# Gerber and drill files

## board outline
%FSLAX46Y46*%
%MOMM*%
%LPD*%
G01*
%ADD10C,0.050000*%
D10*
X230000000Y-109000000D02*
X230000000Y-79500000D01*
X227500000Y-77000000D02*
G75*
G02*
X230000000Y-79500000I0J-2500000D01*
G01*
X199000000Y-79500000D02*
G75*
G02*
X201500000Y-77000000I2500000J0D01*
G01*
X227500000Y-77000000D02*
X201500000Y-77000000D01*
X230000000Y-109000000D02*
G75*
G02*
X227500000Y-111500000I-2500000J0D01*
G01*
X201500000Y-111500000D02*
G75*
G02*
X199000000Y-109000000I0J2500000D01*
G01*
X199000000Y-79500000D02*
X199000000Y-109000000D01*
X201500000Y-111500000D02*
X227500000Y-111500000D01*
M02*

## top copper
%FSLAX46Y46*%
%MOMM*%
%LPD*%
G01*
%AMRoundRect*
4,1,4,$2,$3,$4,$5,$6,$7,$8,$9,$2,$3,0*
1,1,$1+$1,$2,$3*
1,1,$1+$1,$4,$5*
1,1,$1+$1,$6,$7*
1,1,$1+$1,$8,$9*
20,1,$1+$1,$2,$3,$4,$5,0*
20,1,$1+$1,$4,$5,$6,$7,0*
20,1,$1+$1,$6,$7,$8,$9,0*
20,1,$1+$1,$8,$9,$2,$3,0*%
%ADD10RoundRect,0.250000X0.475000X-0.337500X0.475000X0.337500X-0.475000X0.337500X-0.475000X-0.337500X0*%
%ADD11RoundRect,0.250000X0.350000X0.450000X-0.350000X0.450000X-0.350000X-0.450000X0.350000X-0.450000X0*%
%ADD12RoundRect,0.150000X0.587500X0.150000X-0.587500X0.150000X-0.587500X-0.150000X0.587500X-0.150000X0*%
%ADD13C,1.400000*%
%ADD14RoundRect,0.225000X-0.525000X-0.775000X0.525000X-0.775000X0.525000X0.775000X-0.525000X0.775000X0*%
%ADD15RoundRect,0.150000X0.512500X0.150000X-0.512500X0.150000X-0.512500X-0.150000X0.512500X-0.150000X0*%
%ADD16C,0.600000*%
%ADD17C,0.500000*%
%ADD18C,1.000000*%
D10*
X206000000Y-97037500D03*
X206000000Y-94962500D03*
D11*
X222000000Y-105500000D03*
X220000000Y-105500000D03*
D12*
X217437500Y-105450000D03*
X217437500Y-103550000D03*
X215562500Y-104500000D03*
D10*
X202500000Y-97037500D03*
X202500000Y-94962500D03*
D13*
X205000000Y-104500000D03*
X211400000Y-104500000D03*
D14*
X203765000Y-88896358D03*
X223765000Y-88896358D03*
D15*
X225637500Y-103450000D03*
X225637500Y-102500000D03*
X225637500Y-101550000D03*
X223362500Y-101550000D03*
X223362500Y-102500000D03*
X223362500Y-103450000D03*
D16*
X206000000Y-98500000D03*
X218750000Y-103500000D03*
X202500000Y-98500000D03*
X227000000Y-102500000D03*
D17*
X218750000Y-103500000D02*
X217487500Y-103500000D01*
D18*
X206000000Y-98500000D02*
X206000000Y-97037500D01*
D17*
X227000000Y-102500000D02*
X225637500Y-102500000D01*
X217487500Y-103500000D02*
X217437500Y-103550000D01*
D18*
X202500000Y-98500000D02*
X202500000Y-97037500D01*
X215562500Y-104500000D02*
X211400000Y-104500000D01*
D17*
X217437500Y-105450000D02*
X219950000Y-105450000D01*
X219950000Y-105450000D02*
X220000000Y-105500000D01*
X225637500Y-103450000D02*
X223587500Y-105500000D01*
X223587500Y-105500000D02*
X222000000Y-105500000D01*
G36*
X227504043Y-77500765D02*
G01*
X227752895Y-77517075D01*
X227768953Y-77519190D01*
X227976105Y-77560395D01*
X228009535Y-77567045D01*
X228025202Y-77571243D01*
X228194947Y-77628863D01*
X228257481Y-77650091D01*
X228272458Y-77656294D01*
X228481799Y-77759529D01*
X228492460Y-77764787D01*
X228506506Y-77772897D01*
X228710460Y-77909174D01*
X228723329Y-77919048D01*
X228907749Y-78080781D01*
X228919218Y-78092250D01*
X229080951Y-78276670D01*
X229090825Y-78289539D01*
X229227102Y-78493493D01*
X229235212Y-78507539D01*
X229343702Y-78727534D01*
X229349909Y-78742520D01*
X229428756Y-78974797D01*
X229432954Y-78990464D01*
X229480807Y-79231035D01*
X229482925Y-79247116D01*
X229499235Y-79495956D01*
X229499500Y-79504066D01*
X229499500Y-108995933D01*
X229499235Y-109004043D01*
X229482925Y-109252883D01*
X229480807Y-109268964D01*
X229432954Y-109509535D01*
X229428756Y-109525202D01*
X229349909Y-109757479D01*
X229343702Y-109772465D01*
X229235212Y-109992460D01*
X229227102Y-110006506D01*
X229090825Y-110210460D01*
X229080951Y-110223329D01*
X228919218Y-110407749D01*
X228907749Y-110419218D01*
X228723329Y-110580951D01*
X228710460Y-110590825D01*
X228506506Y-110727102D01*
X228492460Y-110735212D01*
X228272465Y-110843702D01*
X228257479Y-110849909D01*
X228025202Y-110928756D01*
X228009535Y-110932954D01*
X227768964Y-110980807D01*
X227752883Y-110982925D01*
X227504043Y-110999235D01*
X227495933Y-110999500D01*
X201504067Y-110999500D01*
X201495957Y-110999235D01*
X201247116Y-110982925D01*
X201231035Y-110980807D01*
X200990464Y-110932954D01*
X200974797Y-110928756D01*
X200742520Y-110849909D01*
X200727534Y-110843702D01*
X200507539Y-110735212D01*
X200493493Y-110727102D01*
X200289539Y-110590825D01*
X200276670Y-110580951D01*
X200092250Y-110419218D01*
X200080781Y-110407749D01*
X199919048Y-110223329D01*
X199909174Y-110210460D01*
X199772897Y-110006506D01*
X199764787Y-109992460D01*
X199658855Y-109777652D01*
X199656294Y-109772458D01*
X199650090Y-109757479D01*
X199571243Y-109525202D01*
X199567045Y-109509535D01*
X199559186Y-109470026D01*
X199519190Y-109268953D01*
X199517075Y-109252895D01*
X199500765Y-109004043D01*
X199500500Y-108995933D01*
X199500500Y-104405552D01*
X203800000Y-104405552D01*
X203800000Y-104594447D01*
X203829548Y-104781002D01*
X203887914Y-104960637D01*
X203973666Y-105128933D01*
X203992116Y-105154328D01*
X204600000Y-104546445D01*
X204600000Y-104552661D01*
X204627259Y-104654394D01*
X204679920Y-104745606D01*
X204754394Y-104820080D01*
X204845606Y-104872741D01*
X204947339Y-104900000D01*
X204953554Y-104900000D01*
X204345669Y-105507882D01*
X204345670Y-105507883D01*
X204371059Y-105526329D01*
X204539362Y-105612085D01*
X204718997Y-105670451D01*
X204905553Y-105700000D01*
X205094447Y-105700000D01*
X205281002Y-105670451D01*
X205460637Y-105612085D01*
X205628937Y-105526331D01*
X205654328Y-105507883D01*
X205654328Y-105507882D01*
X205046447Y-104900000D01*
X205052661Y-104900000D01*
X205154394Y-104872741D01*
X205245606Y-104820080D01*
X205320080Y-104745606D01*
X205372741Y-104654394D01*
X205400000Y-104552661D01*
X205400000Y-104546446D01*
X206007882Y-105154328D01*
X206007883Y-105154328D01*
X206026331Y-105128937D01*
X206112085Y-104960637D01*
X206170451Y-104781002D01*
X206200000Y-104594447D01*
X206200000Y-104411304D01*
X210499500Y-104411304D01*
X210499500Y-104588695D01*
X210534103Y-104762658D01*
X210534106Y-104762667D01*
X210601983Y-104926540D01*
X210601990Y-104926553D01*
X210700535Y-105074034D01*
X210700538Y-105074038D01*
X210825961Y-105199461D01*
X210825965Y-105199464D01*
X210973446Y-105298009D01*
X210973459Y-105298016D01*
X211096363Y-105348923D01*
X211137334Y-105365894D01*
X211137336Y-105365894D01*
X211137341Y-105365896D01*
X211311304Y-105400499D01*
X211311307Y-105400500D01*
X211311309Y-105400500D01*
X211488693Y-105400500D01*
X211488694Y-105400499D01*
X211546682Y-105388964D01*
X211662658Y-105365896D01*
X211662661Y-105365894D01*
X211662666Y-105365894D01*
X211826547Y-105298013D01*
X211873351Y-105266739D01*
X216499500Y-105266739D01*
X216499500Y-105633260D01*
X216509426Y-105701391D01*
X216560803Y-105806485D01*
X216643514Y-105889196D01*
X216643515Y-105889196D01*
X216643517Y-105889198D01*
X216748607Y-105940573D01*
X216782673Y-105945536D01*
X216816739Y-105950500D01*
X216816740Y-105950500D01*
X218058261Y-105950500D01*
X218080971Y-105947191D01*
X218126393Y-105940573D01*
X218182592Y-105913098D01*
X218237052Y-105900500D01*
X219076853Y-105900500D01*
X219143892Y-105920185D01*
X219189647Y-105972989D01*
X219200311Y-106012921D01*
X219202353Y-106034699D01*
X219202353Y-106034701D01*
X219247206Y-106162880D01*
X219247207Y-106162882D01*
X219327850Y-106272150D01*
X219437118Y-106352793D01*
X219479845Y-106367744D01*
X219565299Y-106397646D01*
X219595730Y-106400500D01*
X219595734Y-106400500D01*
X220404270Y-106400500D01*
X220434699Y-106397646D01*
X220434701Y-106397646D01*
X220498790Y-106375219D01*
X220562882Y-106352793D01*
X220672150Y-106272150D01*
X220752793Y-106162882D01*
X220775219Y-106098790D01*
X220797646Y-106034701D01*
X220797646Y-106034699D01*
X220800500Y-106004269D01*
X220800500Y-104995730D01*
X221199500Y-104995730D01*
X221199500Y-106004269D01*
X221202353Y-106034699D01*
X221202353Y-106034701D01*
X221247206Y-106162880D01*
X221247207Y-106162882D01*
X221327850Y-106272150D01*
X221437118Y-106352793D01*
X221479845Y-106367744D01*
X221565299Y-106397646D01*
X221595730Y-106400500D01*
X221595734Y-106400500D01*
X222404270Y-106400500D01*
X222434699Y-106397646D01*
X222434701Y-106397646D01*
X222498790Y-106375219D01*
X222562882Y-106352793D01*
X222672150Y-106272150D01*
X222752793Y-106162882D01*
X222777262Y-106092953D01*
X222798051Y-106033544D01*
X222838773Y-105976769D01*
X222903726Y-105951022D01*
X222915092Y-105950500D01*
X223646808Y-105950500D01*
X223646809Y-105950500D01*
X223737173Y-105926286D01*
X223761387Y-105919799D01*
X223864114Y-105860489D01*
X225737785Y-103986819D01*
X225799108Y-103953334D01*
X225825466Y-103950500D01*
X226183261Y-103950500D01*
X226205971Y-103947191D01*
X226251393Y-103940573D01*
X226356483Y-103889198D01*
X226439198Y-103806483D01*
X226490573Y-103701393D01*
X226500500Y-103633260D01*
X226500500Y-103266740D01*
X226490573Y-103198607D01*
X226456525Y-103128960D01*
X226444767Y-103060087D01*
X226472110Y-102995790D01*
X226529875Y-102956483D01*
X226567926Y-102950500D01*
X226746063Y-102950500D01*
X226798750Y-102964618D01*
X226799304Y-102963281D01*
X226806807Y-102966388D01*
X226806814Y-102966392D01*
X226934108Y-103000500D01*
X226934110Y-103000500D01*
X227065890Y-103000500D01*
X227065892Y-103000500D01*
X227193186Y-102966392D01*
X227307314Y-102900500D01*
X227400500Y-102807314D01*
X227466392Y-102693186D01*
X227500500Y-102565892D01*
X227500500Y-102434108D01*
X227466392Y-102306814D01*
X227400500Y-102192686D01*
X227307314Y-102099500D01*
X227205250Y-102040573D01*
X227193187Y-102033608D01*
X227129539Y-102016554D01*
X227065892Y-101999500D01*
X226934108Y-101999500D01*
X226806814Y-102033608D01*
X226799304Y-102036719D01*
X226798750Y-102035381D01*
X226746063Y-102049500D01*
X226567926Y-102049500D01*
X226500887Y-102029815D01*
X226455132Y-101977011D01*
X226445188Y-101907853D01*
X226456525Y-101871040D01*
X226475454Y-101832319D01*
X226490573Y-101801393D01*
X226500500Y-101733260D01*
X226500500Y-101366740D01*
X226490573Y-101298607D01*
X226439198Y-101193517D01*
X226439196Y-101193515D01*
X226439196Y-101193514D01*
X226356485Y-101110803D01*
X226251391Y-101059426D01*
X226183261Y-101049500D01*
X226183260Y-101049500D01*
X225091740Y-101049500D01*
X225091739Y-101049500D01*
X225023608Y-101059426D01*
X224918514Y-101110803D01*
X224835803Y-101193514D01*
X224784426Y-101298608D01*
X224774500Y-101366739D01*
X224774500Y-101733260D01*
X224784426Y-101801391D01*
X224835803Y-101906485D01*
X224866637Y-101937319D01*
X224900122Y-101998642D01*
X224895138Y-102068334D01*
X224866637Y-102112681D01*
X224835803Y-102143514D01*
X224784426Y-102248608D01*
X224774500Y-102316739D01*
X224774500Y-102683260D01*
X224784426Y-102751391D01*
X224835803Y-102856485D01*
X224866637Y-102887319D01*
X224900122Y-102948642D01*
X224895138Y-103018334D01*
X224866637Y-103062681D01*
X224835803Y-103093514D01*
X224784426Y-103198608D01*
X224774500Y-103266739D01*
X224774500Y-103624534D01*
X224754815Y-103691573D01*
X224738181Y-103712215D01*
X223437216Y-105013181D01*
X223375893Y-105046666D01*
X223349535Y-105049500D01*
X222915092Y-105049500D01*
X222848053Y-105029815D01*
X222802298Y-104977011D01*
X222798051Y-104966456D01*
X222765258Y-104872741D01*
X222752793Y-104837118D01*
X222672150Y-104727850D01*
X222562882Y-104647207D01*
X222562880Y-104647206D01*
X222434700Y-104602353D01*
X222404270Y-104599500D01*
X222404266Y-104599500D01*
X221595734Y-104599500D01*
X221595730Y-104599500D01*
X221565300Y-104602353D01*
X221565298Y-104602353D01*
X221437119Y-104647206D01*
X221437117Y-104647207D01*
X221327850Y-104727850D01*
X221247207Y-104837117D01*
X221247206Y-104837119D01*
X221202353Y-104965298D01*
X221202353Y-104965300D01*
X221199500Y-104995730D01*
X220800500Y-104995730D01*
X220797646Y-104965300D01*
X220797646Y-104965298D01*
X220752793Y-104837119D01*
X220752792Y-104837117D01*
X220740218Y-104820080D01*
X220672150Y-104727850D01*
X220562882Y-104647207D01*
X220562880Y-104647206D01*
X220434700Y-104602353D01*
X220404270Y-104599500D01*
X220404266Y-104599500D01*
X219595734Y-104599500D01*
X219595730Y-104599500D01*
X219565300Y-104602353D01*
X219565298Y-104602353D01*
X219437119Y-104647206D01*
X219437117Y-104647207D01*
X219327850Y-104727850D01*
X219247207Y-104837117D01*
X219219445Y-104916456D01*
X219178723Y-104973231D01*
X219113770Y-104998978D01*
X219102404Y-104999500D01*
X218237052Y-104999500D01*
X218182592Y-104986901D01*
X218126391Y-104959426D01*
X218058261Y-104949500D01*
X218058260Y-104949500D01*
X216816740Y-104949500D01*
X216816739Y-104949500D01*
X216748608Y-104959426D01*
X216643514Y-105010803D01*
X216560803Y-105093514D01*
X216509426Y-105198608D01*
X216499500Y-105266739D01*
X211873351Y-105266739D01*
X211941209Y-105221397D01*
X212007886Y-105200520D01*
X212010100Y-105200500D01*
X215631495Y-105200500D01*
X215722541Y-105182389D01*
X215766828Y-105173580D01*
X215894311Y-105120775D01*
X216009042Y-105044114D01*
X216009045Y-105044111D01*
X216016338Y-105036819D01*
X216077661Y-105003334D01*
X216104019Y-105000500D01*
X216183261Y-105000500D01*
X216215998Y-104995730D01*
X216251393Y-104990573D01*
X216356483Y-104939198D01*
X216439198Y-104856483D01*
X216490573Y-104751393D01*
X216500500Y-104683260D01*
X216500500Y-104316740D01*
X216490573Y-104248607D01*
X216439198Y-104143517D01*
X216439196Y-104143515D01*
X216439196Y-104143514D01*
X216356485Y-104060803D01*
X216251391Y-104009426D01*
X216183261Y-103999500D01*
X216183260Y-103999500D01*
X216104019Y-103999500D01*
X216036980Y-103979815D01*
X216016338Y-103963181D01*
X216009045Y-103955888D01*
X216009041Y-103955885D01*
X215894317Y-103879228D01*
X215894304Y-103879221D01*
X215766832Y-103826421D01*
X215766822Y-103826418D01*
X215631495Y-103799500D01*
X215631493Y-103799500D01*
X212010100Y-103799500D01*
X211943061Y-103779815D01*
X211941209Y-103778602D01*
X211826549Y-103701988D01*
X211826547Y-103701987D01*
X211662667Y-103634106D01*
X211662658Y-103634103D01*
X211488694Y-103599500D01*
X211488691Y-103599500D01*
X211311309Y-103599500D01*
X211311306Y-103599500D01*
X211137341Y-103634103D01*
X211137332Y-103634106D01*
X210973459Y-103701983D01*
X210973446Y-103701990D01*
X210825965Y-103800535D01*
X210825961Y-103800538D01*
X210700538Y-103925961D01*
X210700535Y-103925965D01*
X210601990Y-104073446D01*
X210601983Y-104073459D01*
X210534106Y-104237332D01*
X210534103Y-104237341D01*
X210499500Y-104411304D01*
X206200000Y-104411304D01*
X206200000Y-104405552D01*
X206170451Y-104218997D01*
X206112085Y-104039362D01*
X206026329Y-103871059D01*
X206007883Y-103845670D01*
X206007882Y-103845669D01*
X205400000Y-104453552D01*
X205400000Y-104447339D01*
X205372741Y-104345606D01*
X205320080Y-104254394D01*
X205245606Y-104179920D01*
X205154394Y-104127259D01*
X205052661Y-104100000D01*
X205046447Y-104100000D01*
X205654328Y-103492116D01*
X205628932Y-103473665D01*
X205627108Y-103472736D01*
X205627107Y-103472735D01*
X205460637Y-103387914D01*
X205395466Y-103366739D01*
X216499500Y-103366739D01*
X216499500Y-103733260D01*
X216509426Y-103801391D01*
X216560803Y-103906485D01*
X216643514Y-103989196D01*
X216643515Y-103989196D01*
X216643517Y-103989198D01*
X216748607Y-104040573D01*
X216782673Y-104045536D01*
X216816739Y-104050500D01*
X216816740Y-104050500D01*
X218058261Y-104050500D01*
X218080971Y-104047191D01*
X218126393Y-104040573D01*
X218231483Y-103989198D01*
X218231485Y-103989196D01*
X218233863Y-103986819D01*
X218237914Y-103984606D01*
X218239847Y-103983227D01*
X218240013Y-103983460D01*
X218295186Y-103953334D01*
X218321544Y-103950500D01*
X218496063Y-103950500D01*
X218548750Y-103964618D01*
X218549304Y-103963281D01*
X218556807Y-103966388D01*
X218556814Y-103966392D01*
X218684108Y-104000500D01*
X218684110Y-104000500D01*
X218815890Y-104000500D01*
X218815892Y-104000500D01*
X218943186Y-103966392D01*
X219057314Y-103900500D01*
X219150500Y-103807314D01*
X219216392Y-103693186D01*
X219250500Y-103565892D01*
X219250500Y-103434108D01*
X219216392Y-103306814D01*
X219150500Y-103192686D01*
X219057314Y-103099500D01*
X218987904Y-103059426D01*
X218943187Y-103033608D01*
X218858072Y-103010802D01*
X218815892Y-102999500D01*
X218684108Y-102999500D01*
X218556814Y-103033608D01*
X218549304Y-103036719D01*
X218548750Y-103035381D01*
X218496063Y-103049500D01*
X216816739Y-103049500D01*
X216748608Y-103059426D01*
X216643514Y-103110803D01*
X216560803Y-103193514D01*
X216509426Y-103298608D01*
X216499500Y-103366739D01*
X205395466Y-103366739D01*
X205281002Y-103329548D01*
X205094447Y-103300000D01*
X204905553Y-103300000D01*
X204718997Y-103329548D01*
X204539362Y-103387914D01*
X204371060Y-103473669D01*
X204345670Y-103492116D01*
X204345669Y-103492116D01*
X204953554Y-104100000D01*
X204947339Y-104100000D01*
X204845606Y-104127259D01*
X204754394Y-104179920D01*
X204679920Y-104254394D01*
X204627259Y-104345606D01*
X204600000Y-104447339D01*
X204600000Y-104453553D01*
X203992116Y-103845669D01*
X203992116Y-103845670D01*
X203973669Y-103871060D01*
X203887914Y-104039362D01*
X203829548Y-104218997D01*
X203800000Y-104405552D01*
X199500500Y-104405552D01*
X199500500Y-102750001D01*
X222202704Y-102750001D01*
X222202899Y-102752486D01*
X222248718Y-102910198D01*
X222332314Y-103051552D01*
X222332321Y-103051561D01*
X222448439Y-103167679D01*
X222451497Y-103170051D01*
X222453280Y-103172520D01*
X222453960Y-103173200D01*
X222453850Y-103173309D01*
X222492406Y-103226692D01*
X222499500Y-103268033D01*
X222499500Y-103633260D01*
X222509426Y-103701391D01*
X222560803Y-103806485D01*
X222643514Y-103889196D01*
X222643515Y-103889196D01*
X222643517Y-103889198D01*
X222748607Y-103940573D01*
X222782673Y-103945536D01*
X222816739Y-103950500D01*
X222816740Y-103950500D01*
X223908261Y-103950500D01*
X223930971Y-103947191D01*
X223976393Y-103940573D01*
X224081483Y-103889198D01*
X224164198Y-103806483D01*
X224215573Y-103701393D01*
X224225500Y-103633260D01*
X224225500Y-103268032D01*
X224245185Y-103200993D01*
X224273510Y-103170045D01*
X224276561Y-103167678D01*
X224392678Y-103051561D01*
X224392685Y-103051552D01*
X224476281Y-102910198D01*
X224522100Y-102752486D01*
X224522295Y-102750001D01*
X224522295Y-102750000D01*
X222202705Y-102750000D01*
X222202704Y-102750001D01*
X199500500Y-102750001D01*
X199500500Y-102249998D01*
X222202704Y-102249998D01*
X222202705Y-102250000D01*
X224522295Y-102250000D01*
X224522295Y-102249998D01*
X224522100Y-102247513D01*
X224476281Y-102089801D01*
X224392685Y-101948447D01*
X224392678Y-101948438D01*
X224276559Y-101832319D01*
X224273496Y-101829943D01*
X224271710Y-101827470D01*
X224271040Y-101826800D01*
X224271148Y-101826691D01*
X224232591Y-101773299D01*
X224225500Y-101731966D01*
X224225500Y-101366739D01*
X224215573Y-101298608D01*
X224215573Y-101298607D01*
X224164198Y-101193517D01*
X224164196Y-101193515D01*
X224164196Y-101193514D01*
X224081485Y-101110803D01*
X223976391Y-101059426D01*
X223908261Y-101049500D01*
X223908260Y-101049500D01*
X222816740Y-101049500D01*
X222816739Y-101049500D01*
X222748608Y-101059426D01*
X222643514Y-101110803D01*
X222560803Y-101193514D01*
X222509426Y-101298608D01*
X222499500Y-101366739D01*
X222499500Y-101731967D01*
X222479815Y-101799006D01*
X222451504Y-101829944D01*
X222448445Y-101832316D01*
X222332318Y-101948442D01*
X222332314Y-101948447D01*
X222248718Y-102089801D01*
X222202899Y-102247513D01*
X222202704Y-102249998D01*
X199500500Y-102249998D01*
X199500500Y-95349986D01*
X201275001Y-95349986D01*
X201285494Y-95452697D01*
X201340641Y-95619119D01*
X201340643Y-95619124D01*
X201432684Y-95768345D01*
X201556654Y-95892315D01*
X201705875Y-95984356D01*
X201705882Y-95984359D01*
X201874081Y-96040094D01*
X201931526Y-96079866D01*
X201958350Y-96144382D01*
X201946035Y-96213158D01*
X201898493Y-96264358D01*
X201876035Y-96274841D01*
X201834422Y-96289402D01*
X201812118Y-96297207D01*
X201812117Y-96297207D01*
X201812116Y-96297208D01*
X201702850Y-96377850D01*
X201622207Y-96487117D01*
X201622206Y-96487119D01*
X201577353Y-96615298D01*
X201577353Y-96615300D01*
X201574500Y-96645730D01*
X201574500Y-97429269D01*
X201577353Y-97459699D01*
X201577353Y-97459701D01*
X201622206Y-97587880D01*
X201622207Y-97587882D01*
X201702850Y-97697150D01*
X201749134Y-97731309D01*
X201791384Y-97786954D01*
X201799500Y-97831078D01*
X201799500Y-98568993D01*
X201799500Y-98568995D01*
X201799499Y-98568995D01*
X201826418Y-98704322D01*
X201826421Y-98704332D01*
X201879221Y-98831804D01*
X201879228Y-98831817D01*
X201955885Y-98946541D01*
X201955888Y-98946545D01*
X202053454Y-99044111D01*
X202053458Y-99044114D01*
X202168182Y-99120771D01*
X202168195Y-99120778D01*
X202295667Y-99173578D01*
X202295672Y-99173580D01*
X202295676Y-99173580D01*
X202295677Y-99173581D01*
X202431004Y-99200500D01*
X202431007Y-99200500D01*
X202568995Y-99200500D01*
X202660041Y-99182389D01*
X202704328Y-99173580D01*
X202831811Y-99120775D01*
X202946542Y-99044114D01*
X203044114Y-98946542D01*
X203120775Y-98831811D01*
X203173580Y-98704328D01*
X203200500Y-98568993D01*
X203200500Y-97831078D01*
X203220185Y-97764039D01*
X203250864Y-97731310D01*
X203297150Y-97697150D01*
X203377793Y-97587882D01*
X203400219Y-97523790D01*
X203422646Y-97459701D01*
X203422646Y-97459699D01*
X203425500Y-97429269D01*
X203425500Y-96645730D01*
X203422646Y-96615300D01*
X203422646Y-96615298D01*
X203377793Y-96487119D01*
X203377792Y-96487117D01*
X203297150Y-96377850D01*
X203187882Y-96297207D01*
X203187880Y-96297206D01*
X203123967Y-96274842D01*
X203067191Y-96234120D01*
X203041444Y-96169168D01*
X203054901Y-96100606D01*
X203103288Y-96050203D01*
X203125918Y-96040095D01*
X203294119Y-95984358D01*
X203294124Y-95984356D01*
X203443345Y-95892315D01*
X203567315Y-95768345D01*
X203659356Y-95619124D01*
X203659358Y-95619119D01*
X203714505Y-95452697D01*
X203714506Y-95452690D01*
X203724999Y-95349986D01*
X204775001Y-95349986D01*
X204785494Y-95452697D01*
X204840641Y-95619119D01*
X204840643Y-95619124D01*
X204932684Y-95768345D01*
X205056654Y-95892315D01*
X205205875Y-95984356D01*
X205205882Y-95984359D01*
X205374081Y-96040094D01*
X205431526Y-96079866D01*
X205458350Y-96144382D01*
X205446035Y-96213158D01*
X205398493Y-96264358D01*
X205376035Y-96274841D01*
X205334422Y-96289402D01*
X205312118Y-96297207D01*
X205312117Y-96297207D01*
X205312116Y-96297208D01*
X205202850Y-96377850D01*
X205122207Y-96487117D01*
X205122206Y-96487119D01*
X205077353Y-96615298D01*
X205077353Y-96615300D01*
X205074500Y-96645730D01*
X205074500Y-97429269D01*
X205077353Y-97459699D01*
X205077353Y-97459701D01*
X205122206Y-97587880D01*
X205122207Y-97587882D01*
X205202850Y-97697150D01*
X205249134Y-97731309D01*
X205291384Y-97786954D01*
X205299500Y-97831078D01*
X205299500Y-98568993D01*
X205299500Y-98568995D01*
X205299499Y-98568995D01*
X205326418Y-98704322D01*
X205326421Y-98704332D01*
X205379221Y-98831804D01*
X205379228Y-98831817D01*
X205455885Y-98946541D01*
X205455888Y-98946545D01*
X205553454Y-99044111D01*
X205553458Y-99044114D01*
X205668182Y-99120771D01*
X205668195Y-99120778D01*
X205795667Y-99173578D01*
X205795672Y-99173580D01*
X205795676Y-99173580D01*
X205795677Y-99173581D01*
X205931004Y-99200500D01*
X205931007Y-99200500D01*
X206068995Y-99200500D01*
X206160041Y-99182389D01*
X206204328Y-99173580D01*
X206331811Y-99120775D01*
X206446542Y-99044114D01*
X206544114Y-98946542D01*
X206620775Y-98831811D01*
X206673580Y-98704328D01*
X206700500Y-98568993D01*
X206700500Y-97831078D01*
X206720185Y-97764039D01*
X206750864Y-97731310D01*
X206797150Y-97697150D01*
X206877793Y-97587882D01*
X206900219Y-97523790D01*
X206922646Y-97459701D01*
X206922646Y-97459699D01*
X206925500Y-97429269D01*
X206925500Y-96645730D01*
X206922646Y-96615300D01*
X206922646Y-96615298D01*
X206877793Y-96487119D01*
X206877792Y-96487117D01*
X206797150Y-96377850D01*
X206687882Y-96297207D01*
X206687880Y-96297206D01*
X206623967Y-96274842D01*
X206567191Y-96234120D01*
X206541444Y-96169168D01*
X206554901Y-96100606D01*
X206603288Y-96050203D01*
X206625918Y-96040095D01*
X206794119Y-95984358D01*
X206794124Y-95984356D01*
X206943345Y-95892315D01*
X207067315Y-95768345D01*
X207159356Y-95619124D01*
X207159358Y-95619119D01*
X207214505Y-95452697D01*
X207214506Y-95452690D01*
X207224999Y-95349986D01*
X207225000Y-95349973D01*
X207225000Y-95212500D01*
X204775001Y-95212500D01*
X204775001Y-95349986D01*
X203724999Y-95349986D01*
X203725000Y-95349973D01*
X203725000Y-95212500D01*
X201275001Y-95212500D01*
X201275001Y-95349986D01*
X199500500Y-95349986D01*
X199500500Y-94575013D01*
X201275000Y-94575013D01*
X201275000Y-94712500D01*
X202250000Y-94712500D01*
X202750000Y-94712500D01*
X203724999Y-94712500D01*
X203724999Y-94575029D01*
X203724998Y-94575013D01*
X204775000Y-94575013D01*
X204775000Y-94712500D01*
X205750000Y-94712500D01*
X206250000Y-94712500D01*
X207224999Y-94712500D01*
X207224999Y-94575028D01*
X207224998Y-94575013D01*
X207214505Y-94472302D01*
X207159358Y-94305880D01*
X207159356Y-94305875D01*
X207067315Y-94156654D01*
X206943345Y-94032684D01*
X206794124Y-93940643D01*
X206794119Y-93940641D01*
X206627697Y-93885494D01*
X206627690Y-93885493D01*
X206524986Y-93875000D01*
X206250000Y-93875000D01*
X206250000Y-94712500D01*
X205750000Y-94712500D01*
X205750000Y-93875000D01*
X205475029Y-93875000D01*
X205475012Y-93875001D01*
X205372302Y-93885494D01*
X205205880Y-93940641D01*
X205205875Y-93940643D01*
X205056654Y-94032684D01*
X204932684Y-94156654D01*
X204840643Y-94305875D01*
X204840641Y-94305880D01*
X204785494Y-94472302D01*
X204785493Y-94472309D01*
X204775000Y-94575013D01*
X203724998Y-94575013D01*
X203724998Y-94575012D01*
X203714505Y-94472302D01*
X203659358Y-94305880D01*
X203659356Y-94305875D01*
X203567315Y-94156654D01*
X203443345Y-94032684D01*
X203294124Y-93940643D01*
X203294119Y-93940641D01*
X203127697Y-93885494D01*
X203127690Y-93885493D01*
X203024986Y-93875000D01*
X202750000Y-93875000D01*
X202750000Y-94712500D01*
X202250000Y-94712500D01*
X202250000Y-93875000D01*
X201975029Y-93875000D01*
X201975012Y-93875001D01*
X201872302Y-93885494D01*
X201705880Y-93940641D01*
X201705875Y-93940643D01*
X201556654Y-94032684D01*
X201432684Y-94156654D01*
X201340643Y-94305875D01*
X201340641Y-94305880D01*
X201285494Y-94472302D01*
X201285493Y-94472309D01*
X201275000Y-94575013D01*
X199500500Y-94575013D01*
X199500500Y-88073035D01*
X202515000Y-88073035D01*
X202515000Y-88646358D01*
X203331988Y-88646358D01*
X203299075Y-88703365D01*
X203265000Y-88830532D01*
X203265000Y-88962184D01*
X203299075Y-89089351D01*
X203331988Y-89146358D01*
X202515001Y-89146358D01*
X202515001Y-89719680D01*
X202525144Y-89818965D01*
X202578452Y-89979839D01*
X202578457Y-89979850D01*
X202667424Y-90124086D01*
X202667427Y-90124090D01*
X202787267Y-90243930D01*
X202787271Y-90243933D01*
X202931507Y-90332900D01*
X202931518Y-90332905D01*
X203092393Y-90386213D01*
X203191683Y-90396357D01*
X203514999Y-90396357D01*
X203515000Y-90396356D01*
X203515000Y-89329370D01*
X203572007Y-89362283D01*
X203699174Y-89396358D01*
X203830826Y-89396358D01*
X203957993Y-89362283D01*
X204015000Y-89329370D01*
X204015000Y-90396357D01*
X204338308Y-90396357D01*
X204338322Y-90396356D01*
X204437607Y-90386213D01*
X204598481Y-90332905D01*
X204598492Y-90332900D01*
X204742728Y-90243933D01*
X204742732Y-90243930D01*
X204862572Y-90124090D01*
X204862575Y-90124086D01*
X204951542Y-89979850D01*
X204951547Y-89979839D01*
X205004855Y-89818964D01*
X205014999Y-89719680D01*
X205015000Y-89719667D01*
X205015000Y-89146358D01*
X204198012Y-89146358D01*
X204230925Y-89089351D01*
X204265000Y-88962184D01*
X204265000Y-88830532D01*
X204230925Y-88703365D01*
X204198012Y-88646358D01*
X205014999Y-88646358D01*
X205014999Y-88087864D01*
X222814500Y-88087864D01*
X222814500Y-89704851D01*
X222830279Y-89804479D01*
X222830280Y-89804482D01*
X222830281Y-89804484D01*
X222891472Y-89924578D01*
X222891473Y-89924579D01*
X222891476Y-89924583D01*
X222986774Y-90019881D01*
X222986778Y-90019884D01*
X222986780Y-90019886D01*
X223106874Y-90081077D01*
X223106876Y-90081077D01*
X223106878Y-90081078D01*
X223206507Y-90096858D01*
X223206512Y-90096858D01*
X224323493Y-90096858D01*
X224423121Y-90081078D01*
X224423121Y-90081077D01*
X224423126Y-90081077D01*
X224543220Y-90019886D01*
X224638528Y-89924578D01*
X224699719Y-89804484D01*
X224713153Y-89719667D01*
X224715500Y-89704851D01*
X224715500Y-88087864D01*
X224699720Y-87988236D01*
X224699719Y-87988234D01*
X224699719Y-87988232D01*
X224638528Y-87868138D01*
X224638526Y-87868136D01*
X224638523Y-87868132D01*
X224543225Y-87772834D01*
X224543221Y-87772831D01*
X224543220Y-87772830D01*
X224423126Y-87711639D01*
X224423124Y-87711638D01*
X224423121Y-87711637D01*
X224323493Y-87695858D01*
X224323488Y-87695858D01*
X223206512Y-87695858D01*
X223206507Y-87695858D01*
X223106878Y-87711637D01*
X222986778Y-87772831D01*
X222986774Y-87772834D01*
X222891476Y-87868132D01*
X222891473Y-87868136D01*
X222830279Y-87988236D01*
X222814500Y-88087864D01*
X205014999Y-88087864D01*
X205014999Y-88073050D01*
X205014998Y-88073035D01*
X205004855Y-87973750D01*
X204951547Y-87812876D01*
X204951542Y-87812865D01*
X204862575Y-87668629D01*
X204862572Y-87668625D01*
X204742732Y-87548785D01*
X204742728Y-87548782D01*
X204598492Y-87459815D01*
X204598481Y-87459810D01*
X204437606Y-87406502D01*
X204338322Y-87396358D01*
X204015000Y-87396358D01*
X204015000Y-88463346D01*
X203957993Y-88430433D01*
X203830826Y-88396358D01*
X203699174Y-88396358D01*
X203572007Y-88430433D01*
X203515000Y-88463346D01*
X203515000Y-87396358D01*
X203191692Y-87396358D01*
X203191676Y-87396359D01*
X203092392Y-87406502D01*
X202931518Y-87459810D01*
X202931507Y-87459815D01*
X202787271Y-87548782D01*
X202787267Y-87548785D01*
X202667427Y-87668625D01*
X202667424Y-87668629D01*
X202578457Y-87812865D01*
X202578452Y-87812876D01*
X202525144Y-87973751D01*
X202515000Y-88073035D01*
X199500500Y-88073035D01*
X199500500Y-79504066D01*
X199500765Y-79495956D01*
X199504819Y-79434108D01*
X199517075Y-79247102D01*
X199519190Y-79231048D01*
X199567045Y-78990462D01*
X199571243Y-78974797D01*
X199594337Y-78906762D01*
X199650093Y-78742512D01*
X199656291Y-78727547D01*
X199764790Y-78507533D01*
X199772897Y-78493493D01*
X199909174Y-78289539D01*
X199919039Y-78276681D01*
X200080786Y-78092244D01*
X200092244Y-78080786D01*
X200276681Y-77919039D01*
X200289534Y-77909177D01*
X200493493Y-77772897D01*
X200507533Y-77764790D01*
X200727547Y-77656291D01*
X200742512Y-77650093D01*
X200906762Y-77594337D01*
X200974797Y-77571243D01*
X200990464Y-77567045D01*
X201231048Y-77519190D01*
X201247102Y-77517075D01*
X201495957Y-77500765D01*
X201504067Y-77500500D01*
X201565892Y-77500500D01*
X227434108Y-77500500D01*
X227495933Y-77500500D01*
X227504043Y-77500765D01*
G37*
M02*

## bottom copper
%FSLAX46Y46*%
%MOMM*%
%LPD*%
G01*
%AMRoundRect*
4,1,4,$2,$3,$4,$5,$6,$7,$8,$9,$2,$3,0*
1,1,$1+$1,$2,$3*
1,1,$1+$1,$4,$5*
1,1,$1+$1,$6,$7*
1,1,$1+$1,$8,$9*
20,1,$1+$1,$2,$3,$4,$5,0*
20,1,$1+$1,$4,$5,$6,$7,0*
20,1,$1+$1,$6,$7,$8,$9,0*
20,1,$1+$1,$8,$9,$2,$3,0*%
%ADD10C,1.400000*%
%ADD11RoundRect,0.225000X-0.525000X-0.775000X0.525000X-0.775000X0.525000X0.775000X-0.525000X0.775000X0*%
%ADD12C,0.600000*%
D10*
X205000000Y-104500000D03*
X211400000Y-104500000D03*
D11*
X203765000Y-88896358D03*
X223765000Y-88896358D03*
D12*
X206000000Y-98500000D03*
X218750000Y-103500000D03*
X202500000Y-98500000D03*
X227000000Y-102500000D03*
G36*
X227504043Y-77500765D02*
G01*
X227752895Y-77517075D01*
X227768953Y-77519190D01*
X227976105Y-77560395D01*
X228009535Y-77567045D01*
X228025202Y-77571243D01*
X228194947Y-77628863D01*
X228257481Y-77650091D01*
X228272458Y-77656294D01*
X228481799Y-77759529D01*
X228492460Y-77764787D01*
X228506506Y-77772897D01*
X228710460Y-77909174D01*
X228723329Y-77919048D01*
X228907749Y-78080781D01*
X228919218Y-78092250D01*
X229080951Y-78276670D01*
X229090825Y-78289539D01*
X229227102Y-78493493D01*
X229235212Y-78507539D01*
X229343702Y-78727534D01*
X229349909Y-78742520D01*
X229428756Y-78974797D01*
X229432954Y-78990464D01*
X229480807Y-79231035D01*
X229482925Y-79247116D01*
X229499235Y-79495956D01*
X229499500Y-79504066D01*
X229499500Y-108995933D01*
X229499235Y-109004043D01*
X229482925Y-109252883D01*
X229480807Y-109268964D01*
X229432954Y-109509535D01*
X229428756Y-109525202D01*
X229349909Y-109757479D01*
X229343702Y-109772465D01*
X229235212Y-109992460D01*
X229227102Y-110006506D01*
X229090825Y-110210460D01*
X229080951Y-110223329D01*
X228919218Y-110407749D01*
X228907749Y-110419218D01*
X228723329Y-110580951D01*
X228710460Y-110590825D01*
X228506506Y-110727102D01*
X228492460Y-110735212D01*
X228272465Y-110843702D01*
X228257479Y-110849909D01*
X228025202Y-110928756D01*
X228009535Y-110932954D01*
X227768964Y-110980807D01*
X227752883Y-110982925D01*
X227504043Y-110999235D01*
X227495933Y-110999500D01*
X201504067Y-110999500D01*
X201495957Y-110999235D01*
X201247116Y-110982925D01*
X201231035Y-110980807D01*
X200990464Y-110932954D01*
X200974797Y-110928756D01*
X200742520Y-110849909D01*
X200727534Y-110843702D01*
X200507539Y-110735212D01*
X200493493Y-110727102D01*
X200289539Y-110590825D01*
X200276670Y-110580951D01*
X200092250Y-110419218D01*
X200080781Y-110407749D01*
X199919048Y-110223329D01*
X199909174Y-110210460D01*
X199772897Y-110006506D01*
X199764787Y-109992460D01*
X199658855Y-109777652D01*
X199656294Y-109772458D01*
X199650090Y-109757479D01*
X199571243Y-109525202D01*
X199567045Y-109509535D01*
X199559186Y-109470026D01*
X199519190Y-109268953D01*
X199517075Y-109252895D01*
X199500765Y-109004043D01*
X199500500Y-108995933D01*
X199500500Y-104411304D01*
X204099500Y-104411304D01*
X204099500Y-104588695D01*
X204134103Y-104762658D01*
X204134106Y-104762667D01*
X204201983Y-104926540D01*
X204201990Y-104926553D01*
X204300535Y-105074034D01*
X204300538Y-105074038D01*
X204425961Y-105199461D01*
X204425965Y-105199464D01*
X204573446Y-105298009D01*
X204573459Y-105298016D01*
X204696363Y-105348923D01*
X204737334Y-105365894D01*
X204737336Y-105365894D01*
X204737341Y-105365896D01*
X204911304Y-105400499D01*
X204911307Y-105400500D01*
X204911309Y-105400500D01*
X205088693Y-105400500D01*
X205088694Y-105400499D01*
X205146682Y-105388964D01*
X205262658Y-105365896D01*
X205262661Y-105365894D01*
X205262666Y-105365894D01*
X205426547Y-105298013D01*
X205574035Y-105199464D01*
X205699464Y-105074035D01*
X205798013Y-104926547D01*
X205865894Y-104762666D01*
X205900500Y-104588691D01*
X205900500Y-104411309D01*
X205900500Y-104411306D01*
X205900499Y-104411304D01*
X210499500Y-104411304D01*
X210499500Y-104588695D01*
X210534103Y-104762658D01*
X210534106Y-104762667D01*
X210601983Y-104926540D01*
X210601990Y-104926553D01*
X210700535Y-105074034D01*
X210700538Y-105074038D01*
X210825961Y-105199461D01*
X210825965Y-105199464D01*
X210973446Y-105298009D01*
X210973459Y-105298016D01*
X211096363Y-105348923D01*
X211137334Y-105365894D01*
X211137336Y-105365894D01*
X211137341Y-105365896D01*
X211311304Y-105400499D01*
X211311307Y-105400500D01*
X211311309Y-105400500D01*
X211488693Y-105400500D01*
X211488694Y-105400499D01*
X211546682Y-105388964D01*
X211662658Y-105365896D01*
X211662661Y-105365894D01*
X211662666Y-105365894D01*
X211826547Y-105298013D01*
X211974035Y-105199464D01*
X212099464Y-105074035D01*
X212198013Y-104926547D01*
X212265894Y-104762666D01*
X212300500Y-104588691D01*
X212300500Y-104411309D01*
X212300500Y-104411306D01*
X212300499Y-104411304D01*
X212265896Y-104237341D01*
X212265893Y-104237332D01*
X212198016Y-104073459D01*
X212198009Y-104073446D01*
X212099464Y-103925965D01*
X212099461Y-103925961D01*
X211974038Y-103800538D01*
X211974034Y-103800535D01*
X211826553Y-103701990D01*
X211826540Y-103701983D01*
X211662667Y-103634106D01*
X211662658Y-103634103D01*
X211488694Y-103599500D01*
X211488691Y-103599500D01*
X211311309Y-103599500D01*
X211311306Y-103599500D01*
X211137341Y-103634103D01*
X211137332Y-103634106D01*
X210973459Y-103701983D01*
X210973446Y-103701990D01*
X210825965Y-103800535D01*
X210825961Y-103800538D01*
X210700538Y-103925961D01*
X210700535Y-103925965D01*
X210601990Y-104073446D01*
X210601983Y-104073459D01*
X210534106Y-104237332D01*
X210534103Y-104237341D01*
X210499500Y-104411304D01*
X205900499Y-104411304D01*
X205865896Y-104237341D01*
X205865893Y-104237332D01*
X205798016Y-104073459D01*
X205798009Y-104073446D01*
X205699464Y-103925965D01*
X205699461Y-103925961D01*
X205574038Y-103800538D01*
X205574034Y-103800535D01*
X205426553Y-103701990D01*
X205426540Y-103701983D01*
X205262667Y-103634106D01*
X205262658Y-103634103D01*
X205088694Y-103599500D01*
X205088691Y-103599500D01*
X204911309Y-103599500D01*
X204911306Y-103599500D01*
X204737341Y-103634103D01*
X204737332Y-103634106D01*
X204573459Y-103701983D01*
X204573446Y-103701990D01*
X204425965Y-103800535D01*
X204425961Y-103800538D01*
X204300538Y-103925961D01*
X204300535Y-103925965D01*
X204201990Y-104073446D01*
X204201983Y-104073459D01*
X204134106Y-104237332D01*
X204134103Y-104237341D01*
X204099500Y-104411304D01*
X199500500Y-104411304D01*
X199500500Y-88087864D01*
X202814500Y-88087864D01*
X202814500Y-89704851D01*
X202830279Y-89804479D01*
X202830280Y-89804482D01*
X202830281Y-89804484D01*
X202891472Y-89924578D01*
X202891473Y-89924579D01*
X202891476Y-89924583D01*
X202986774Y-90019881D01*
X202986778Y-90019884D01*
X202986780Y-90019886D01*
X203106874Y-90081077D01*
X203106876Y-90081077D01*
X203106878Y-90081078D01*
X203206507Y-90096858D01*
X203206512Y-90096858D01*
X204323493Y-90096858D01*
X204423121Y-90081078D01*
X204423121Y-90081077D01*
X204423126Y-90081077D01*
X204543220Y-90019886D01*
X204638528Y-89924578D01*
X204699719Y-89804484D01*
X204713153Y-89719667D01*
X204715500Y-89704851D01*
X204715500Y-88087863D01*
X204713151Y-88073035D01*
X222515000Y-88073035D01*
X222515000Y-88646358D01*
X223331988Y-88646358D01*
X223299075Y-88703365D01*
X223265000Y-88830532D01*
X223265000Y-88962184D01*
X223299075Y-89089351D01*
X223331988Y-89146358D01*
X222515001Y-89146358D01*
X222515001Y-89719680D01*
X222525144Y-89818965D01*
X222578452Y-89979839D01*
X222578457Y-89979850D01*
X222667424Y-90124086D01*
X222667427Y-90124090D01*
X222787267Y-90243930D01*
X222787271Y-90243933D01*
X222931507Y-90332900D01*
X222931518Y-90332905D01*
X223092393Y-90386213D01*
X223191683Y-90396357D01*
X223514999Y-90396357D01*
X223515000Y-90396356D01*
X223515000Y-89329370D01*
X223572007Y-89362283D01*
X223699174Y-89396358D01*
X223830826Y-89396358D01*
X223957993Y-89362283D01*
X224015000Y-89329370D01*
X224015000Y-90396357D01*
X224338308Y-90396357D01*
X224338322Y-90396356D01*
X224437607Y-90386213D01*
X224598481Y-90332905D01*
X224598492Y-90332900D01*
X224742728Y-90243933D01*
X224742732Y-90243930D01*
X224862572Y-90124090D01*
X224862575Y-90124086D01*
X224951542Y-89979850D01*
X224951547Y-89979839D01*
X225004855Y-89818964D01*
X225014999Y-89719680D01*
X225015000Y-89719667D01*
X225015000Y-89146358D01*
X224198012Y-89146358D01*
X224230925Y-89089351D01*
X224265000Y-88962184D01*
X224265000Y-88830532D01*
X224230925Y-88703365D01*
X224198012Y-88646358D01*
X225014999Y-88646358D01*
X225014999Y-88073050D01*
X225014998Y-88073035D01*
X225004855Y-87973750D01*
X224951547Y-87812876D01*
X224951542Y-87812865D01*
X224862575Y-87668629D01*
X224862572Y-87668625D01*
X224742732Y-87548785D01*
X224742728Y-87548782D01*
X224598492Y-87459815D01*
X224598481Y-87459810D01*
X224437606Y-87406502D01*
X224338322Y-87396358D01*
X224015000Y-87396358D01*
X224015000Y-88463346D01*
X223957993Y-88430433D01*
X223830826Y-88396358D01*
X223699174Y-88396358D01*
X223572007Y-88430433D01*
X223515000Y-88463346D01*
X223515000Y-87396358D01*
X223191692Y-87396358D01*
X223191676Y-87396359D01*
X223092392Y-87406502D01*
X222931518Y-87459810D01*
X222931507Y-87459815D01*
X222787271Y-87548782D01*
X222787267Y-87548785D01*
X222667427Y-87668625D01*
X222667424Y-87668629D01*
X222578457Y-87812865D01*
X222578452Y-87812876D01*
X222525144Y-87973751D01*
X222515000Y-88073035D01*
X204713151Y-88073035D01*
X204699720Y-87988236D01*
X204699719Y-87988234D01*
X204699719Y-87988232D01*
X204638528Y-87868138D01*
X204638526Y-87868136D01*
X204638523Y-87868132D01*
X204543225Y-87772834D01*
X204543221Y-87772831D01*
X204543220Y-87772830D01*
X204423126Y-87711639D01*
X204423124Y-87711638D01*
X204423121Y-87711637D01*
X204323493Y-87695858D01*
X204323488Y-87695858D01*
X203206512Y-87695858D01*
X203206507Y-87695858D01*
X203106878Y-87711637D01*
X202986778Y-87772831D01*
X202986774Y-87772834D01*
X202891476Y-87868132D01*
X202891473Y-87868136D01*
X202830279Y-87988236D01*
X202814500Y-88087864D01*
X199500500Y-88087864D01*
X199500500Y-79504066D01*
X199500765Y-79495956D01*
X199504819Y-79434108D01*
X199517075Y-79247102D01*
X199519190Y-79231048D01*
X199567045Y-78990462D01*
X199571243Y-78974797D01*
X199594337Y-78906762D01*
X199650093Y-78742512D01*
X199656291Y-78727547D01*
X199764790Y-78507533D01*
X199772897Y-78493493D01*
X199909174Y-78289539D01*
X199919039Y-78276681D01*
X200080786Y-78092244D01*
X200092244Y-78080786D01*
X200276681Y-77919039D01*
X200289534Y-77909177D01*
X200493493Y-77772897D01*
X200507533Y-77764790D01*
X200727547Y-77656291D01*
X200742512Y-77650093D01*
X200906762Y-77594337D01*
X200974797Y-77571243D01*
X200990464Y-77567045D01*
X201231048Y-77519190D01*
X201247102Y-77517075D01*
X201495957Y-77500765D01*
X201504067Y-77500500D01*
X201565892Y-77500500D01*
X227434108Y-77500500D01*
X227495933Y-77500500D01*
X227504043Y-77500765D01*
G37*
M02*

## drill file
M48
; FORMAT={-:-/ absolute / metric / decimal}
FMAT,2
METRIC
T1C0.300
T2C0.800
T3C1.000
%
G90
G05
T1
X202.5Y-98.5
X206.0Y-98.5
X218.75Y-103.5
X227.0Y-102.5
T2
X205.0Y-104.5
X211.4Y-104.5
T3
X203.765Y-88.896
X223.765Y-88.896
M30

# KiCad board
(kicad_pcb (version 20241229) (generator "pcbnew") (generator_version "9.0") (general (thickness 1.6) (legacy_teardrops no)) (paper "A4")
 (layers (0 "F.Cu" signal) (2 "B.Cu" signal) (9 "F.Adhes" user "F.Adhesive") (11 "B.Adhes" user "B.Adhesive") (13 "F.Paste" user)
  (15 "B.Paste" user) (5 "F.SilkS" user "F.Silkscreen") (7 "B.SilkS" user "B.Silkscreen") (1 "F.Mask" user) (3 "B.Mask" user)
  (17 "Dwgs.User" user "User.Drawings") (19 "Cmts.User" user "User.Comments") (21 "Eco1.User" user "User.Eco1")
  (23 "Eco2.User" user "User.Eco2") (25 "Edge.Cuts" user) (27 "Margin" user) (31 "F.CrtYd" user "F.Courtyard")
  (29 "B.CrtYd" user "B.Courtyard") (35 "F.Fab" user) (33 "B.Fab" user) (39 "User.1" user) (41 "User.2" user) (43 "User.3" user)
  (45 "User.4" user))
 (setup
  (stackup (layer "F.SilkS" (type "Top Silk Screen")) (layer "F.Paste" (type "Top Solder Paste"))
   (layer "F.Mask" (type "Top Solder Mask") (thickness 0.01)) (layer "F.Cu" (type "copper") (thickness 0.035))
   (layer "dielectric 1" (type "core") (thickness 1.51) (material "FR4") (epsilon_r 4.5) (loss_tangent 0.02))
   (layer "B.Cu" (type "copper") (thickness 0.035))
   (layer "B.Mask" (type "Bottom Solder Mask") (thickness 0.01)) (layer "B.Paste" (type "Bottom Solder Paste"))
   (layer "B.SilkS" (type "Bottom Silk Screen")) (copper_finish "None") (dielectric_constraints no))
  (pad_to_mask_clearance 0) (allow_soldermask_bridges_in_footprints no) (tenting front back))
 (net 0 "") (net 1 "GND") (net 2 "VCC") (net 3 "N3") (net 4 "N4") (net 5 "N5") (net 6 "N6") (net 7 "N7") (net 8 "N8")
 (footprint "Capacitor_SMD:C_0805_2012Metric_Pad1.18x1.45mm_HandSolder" (layer "F.Cu") (at 206 96 90)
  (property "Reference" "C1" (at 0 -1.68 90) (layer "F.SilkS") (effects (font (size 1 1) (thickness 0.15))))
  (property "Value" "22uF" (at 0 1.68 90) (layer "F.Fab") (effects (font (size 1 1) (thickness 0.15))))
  (pad "1" smd roundrect (at -1.0375 0 90) (size 1.175 1.45) (layers "F.Cu" "F.Mask" "F.Paste") (roundrect_rratio 0.212766) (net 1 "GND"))
  (pad "2" smd roundrect (at 1.0375 0 90) (size 1.175 1.45) (layers "F.Cu" "F.Mask" "F.Paste") (roundrect_rratio 0.212766) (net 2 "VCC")))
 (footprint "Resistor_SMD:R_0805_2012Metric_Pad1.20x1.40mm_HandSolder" (layer "F.Cu") (at 221 105.5 180)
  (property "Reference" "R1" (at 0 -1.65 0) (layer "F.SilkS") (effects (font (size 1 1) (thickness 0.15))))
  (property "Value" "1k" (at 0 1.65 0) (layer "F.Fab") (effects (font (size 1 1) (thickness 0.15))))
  (pad "1" smd roundrect (at -1 0 180) (size 1.2 1.4) (layers "F.Cu" "F.Mask" "F.Paste") (roundrect_rratio 0.208333) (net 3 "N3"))
  (pad "2" smd roundrect (at 1 0 180) (size 1.2 1.4) (layers "F.Cu" "F.Mask" "F.Paste") (roundrect_rratio 0.208333) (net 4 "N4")))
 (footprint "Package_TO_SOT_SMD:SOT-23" (layer "F.Cu") (at 216.5 104.5 180)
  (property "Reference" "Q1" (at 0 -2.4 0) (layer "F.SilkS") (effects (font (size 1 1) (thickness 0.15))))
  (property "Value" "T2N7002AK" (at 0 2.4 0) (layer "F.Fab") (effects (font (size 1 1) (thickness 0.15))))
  (pad "1" smd roundrect (at -0.9375 -0.95 180) (size 1.475 0.6) (layers "F.Cu" "F.Mask" "F.Paste") (roundrect_rratio 0.25) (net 4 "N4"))
  (pad "2" smd roundrect (at -0.9375 0.95 180) (size 1.475 0.6) (layers "F.Cu" "F.Mask" "F.Paste") (roundrect_rratio 0.25) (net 1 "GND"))
  (pad "3" smd roundrect (at 0.9375 0 180) (size 1.475 0.6) (layers "F.Cu" "F.Mask" "F.Paste") (roundrect_rratio 0.25) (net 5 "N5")))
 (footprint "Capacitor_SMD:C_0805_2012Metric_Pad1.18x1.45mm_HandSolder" (layer "F.Cu") (at 202.5 96 90)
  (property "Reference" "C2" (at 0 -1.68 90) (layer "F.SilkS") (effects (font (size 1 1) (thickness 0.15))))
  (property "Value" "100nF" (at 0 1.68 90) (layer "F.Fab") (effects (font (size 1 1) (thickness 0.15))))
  (pad "1" smd roundrect (at -1.0375 0 90) (size 1.175 1.45) (layers "F.Cu" "F.Mask" "F.Paste") (roundrect_rratio 0.212766) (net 1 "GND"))
  (pad "2" smd roundrect (at 1.0375 0 90) (size 1.175 1.45) (layers "F.Cu" "F.Mask" "F.Paste") (roundrect_rratio 0.212766) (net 2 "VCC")))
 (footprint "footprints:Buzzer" (layer "F.Cu") (at 205 104.5)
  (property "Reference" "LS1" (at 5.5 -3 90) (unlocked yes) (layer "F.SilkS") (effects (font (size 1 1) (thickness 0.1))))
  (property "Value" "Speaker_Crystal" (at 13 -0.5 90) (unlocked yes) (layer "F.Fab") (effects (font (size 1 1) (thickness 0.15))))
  (pad "1" thru_hole circle (at 0 0) (size 1.4 1.4) (drill 0.8) (layers "*.Cu" "*.Mask") (remove_unused_layers no) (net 2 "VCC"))
  (pad "2" thru_hole circle (at 6.4 0) (size 1.4 1.4) (drill 0.8) (layers "*.Cu" "*.Mask") (remove_unused_layers no) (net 5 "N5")))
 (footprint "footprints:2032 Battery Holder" (layer "F.Cu") (at 203.765 88.896358)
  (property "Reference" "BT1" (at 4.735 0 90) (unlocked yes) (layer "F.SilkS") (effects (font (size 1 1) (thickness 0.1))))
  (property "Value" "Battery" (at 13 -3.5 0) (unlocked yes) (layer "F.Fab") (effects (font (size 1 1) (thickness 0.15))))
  (pad "1" thru_hole roundrect (at 0 0) (size 1.5 2) (drill 1) (layers "*.Cu" "*.Mask") (remove_unused_layers no) (roundrect_rratio 0.15)
   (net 2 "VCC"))
  (pad "2" thru_hole roundrect (at 20 0) (size 1.5 2) (drill 1) (layers "*.Cu" "*.Mask") (remove_unused_layers no) (roundrect_rratio 0.15)
   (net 1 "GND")))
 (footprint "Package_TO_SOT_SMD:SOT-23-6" (layer "F.Cu") (at 224.5 102.5 180)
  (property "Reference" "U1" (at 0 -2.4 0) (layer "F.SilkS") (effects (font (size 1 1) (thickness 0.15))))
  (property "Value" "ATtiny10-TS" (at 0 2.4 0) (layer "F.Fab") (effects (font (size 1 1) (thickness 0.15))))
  (pad "1" smd roundrect (at -1.1375 -0.95 180) (size 1.325 0.6) (layers "F.Cu" "F.Mask" "F.Paste") (roundrect_rratio 0.25) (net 3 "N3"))
  (pad "2" smd roundrect (at -1.1375 0 180) (size 1.325 0.6) (layers "F.Cu" "F.Mask" "F.Paste") (roundrect_rratio 0.25) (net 1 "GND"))
  (pad "3" smd roundrect (at -1.1375 0.95 180) (size 1.325 0.6) (layers "F.Cu" "F.Mask" "F.Paste") (roundrect_rratio 0.25) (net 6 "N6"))
  (pad "4" smd roundrect (at 1.1375 0.95 180) (size 1.325 0.6) (layers "F.Cu" "F.Mask" "F.Paste") (roundrect_rratio 0.25) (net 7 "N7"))
  (pad "5" smd roundrect (at 1.1375 0 180) (size 1.325 0.6) (layers "F.Cu" "F.Mask" "F.Paste") (roundrect_rratio 0.25) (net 2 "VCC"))
  (pad "6" smd roundrect (at 1.1375 -0.95 180) (size 1.325 0.6) (layers "F.Cu" "F.Mask" "F.Paste") (roundrect_rratio 0.25) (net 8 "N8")))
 (gr_line (start 230 109) (end 230 79.5) (stroke (width 0.05) (type default)) (layer "Edge.Cuts"))
 (gr_arc (start 227.5 77) (mid 229.267767 77.732233) (end 230 79.5) (stroke (width 0.05) (type default)) (layer "Edge.Cuts"))
 (gr_arc (start 199 79.5) (mid 199.732233 77.732233) (end 201.5 77) (stroke (width 0.05) (type default)) (layer "Edge.Cuts"))
 (gr_line (start 227.5 77) (end 201.5 77) (stroke (width 0.05) (type default)) (layer "Edge.Cuts"))
 (gr_arc (start 230 109) (mid 229.267767 110.767767) (end 227.5 111.5) (stroke (width 0.05) (type default)) (layer "Edge.Cuts"))
 (gr_arc (start 201.5 111.5) (mid 199.732233 110.767767) (end 199 109) (stroke (width 0.05) (type default)) (layer "Edge.Cuts"))
 (gr_line (start 199 79.5) (end 199 109) (stroke (width 0.05) (type default)) (layer "Edge.Cuts"))
 (gr_line (start 201.5 111.5) (end 227.5 111.5) (stroke (width 0.05) (type default)) (layer "Edge.Cuts"))
 (segment (start 218.75 103.5) (end 217.4875 103.5) (width 0.5) (layer "F.Cu") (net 1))
 (segment (start 206 98.5) (end 206 97.0375) (width 1) (layer "F.Cu") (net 1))
 (segment (start 227 102.5) (end 225.6375 102.5) (width 0.5) (layer "F.Cu") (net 1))
 (segment (start 217.4875 103.5) (end 217.4375 103.55) (width 0.5) (layer "F.Cu") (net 1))
 (segment (start 202.5 98.5) (end 202.5 97.0375) (width 1) (layer "F.Cu") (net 1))
 (via (at 206 98.5) (size 0.6) (drill 0.3) (layers "F.Cu" "B.Cu") (free yes) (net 1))
 (via (at 218.75 103.5) (size 0.6) (drill 0.3) (layers "F.Cu" "B.Cu") (free yes) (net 1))
 (via (at 202.5 98.5) (size 0.6) (drill 0.3) (layers "F.Cu" "B.Cu") (free yes) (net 1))
 (via (at 227 102.5) (size 0.6) (drill 0.3) (layers "F.Cu" "B.Cu") (free yes) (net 1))
 (segment (start 215.5625 104.5) (end 211.4 104.5) (width 1) (layer "F.Cu") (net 5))
 (segment (start 217.4375 105.45) (end 219.95 105.45) (width 0.5) (layer "F.Cu") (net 4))
 (segment (start 219.95 105.45) (end 220 105.5) (width 0.5) (layer "F.Cu") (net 4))
 (segment (start 225.6375 103.45) (end 223.5875 105.5) (width 0.5) (layer "F.Cu") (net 3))
 (segment (start 223.5875 105.5) (end 222 105.5) (width 0.5) (layer "F.Cu") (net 3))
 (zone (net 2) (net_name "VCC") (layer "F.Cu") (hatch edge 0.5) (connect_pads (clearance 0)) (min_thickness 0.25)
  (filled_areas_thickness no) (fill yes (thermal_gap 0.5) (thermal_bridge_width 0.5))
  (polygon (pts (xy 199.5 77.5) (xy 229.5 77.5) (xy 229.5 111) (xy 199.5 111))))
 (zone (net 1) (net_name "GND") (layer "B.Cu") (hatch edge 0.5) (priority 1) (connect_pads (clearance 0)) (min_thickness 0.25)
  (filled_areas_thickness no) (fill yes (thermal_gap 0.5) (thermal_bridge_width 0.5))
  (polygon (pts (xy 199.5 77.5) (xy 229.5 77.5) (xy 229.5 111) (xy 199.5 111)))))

